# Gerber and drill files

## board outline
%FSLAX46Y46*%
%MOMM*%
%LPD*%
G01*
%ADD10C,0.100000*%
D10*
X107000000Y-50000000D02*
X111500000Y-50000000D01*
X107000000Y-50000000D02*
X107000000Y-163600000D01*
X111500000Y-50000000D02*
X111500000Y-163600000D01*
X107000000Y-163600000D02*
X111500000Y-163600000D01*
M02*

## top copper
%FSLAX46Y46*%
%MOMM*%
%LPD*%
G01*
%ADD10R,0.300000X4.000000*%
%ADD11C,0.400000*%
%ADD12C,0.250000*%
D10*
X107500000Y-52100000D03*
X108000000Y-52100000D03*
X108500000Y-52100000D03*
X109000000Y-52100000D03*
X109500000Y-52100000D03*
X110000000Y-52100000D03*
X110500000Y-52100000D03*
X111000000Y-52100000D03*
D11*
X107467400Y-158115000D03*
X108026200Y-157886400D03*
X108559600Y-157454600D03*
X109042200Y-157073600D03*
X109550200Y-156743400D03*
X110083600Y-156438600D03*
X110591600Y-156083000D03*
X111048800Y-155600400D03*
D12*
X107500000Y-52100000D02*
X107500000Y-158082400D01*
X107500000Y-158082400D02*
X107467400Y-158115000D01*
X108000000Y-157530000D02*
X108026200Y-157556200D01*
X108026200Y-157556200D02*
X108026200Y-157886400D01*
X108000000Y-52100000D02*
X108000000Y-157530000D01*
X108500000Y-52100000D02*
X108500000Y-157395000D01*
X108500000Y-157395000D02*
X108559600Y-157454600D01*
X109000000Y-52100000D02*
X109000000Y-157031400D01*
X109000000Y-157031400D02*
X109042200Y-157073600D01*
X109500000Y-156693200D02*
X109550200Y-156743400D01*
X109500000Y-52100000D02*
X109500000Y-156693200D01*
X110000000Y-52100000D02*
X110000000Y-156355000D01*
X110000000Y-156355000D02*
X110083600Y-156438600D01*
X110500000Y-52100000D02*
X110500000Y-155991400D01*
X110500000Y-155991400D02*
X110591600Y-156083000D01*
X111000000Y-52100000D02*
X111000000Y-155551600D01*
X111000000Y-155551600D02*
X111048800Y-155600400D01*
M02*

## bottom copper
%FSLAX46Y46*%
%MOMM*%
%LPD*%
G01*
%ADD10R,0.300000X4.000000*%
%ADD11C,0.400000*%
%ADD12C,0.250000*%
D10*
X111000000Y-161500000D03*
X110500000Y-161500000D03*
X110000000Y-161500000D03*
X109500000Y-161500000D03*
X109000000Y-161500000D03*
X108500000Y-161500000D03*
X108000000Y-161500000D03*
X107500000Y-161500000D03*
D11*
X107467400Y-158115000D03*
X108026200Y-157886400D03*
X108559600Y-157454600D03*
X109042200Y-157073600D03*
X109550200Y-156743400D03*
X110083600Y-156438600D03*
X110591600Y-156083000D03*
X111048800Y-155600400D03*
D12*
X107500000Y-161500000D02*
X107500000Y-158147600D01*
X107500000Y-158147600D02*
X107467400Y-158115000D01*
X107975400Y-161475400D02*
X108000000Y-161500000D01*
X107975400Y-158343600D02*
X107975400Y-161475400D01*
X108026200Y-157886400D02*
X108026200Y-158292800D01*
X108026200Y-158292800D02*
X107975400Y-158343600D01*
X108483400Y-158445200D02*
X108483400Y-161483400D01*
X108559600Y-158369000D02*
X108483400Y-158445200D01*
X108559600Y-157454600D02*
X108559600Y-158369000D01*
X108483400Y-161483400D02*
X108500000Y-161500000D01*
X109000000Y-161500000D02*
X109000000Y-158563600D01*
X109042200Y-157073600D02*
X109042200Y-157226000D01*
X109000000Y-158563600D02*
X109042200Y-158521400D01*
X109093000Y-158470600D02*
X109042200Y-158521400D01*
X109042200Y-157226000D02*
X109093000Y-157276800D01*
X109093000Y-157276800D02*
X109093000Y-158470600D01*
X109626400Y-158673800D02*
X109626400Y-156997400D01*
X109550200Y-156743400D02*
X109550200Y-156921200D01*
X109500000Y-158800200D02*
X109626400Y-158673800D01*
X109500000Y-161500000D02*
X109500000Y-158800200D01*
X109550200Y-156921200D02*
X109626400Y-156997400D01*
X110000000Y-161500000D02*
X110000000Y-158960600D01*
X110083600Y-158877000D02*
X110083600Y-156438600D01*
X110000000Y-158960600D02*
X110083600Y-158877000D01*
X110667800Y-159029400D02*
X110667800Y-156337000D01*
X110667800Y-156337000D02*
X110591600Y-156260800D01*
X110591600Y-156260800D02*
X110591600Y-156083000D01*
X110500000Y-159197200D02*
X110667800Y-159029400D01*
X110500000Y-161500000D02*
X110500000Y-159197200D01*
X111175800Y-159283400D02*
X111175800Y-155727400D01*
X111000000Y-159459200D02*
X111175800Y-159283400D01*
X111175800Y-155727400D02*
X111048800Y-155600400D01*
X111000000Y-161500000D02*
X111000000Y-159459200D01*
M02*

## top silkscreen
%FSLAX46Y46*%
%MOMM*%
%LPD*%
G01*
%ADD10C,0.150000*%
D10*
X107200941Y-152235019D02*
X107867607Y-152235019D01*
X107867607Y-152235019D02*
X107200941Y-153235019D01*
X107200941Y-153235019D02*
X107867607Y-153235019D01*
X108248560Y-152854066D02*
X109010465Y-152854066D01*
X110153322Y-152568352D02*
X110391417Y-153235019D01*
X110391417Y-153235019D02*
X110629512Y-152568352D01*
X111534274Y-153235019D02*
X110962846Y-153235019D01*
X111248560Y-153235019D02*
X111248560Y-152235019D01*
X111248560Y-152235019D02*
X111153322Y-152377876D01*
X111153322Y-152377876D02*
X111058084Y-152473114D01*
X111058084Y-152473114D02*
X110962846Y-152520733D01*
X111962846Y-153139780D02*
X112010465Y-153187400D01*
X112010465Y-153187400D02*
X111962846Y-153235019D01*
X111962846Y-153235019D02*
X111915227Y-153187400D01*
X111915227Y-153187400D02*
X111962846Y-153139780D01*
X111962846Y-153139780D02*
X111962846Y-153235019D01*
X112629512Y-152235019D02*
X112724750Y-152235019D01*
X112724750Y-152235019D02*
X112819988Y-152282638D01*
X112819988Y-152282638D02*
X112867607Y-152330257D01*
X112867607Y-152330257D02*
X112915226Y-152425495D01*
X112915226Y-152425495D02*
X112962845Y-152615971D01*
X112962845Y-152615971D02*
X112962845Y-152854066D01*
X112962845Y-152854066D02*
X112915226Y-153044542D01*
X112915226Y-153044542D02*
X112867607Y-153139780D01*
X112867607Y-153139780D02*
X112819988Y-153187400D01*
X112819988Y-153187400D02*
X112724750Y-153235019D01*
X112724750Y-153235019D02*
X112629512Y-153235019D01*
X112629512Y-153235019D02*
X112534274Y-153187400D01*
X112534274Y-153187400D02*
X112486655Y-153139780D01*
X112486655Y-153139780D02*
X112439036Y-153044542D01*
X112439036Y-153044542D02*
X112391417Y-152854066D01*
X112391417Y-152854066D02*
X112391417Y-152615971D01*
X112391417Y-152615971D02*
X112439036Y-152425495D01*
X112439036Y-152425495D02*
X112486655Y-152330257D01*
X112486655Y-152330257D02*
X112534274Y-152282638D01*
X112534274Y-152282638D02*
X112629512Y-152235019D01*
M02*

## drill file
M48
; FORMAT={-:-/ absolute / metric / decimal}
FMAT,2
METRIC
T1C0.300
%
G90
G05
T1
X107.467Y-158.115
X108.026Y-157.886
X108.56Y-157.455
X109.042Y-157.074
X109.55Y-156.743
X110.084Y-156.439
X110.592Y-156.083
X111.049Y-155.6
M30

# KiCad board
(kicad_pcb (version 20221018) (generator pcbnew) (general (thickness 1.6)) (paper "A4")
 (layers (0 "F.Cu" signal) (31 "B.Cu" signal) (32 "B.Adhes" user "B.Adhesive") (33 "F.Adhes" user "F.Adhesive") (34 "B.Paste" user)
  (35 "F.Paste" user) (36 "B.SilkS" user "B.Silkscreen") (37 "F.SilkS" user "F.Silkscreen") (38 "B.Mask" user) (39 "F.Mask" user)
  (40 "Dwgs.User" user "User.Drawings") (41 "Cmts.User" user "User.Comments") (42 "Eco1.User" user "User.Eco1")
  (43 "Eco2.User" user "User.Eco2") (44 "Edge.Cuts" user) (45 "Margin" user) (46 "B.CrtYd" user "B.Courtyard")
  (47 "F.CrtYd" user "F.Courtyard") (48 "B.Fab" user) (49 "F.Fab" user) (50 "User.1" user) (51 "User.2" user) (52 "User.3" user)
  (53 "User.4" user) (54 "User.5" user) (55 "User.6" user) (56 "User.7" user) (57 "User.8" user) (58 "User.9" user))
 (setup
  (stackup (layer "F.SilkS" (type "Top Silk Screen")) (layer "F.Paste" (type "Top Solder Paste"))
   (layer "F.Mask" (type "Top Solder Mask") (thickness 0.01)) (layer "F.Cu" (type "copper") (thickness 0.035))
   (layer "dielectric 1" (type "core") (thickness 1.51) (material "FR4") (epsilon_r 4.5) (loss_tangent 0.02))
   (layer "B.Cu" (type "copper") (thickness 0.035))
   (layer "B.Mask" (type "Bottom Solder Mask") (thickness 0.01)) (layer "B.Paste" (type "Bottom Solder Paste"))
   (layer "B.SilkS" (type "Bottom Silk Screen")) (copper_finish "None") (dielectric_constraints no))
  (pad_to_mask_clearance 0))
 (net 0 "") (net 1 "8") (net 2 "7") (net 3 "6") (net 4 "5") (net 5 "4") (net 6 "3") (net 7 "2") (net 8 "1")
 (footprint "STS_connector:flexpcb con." (layer "F.Cu") (at 107 54.1)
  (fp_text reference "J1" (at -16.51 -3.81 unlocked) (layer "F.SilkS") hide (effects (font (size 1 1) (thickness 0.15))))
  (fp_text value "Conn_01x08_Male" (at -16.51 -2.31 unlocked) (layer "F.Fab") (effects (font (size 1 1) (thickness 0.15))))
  (pad "1" smd rect (at 0.5 -2) (size 0.3 4) (layers "F.Cu" "F.Paste" "F.Mask") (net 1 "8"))
  (pad "2" smd rect (at 1 -2) (size 0.3 4) (layers "F.Cu" "F.Paste" "F.Mask") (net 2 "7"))
  (pad "3" smd rect (at 1.5 -2) (size 0.3 4) (layers "F.Cu" "F.Paste" "F.Mask") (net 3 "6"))
  (pad "4" smd rect (at 2 -2) (size 0.3 4) (layers "F.Cu" "F.Paste" "F.Mask") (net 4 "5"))
  (pad "5" smd rect (at 2.5 -2) (size 0.3 4) (layers "F.Cu" "F.Paste" "F.Mask") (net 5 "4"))
  (pad "6" smd rect (at 3 -2) (size 0.3 4) (layers "F.Cu" "F.Paste" "F.Mask") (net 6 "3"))
  (pad "7" smd rect (at 3.5 -2) (size 0.3 4) (layers "F.Cu" "F.Paste" "F.Mask") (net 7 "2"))
  (pad "8" smd rect (at 4 -2) (size 0.3 4) (layers "F.Cu" "F.Paste" "F.Mask") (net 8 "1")))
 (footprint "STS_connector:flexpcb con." (layer "B.Cu") (at 111.5 163.5 180)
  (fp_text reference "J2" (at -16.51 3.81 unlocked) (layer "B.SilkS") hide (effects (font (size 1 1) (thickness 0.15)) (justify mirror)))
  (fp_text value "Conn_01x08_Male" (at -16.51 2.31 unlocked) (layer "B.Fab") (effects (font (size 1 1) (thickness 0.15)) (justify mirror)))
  (pad "1" smd rect (at 0.5 2 180) (size 0.3 4) (layers "B.Cu" "B.Paste" "B.Mask") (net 8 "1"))
  (pad "2" smd rect (at 1 2 180) (size 0.3 4) (layers "B.Cu" "B.Paste" "B.Mask") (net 7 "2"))
  (pad "3" smd rect (at 1.5 2 180) (size 0.3 4) (layers "B.Cu" "B.Paste" "B.Mask") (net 6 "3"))
  (pad "4" smd rect (at 2 2 180) (size 0.3 4) (layers "B.Cu" "B.Paste" "B.Mask") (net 5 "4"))
  (pad "5" smd rect (at 2.5 2 180) (size 0.3 4) (layers "B.Cu" "B.Paste" "B.Mask") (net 4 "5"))
  (pad "6" smd rect (at 3 2 180) (size 0.3 4) (layers "B.Cu" "B.Paste" "B.Mask") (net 3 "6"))
  (pad "7" smd rect (at 3.5 2 180) (size 0.3 4) (layers "B.Cu" "B.Paste" "B.Mask") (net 2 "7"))
  (pad "8" smd rect (at 4 2 180) (size 0.3 4) (layers "B.Cu" "B.Paste" "B.Mask") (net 1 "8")))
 (gr_line (start 107 50) (end 111.5 50) (stroke (width 0.1) (type solid)) (layer "Edge.Cuts"))
 (gr_line (start 107 50) (end 107 163.6) (stroke (width 0.1) (type solid)) (layer "Edge.Cuts"))
 (gr_line (start 111.5 50) (end 111.5 163.6) (stroke (width 0.1) (type solid)) (layer "Edge.Cuts"))
 (gr_line (start 107 163.6) (end 111.5 163.6) (stroke (width 0.1) (type solid)) (layer "Edge.Cuts"))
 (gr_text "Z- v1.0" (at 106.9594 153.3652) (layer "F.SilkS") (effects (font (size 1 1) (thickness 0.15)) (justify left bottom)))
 (segment (start 107.5 52.1) (end 107.5 158.0824) (width 0.25) (layer "F.Cu") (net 1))
 (segment (start 107.5 158.0824) (end 107.4674 158.115) (width 0.25) (layer "F.Cu") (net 1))
 (via (at 107.4674 158.115) (size 0.4) (drill 0.3) (layers "F.Cu" "B.Cu") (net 1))
 (segment (start 107.5 161.5) (end 107.5 158.1476) (width 0.25) (layer "B.Cu") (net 1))
 (segment (start 107.5 158.1476) (end 107.4674 158.115) (width 0.25) (layer "B.Cu") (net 1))
 (segment (start 108 157.53) (end 108.0262 157.5562) (width 0.25) (layer "F.Cu") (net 2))
 (segment (start 108.0262 157.5562) (end 108.0262 157.8864) (width 0.25) (layer "F.Cu") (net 2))
 (segment (start 108 52.1) (end 108 157.53) (width 0.25) (layer "F.Cu") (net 2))
 (via (at 108.0262 157.8864) (size 0.4) (drill 0.3) (layers "F.Cu" "B.Cu") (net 2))
 (segment (start 107.9754 161.4754) (end 108 161.5) (width 0.25) (layer "B.Cu") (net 2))
 (segment (start 107.9754 158.3436) (end 107.9754 161.4754) (width 0.25) (layer "B.Cu") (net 2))
 (segment (start 108.0262 157.8864) (end 108.0262 158.2928) (width 0.25) (layer "B.Cu") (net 2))
 (segment (start 108.0262 158.2928) (end 107.9754 158.3436) (width 0.25) (layer "B.Cu") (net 2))
 (segment (start 108.5 52.1) (end 108.5 157.395) (width 0.25) (layer "F.Cu") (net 3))
 (segment (start 108.5 157.395) (end 108.5596 157.4546) (width 0.25) (layer "F.Cu") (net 3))
 (via (at 108.5596 157.4546) (size 0.4) (drill 0.3) (layers "F.Cu" "B.Cu") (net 3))
 (segment (start 108.4834 158.4452) (end 108.4834 161.4834) (width 0.25) (layer "B.Cu") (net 3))
 (segment (start 108.5596 158.369) (end 108.4834 158.4452) (width 0.25) (layer "B.Cu") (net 3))
 (segment (start 108.5596 157.4546) (end 108.5596 158.369) (width 0.25) (layer "B.Cu") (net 3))
 (segment (start 108.4834 161.4834) (end 108.5 161.5) (width 0.25) (layer "B.Cu") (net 3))
 (segment (start 109 52.1) (end 109 157.0314) (width 0.25) (layer "F.Cu") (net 4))
 (segment (start 109 157.0314) (end 109.0422 157.0736) (width 0.25) (layer "F.Cu") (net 4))
 (via (at 109.0422 157.0736) (size 0.4) (drill 0.3) (layers "F.Cu" "B.Cu") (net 4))
 (segment (start 109 161.5) (end 109 158.5636) (width 0.25) (layer "B.Cu") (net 4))
 (segment (start 109.0422 157.0736) (end 109.0422 157.226) (width 0.25) (layer "B.Cu") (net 4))
 (segment (start 109 158.5636) (end 109.0422 158.5214) (width 0.25) (layer "B.Cu") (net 4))
 (segment (start 109.093 158.4706) (end 109.0422 158.5214) (width 0.25) (layer "B.Cu") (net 4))
 (segment (start 109.0422 157.226) (end 109.093 157.2768) (width 0.25) (layer "B.Cu") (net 4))
 (segment (start 109.093 157.2768) (end 109.093 158.4706) (width 0.25) (layer "B.Cu") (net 4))
 (segment (start 109.5 156.6932) (end 109.5502 156.7434) (width 0.25) (layer "F.Cu") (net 5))
 (segment (start 109.5 52.1) (end 109.5 156.6932) (width 0.25) (layer "F.Cu") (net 5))
 (via (at 109.5502 156.7434) (size 0.4) (drill 0.3) (layers "F.Cu" "B.Cu") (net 5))
 (segment (start 109.6264 158.6738) (end 109.6264 156.9974) (width 0.25) (layer "B.Cu") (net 5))
 (segment (start 109.5502 156.7434) (end 109.5502 156.9212) (width 0.25) (layer "B.Cu") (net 5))
 (segment (start 109.5 158.8002) (end 109.6264 158.6738) (width 0.25) (layer "B.Cu") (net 5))
 (segment (start 109.5 161.5) (end 109.5 158.8002) (width 0.25) (layer "B.Cu") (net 5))
 (segment (start 109.5502 156.9212) (end 109.6264 156.9974) (width 0.25) (layer "B.Cu") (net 5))
 (segment (start 110 52.1) (end 110 156.355) (width 0.25) (layer "F.Cu") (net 6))
 (segment (start 110 156.355) (end 110.0836 156.4386) (width 0.25) (layer "F.Cu") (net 6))
 (via (at 110.0836 156.4386) (size 0.4) (drill 0.3) (layers "F.Cu" "B.Cu") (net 6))
 (segment (start 110 161.5) (end 110 158.9606) (width 0.25) (layer "B.Cu") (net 6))
 (segment (start 110.0836 158.877) (end 110.0836 156.4386) (width 0.25) (layer "B.Cu") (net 6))
 (segment (start 110 158.9606) (end 110.0836 158.877) (width 0.25) (layer "B.Cu") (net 6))
 (segment (start 110.5 52.1) (end 110.5 155.9914) (width 0.25) (layer "F.Cu") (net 7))
 (segment (start 110.5 155.9914) (end 110.5916 156.083) (width 0.25) (layer "F.Cu") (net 7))
 (via (at 110.5916 156.083) (size 0.4) (drill 0.3) (layers "F.Cu" "B.Cu") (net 7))
 (segment (start 110.6678 159.0294) (end 110.6678 156.337) (width 0.25) (layer "B.Cu") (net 7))
 (segment (start 110.6678 156.337) (end 110.5916 156.2608) (width 0.25) (layer "B.Cu") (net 7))
 (segment (start 110.5916 156.2608) (end 110.5916 156.083) (width 0.25) (layer "B.Cu") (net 7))
 (segment (start 110.5 159.1972) (end 110.6678 159.0294) (width 0.25) (layer "B.Cu") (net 7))
 (segment (start 110.5 161.5) (end 110.5 159.1972) (width 0.25) (layer "B.Cu") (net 7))
 (segment (start 111 52.1) (end 111 155.5516) (width 0.25) (layer "F.Cu") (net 8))
 (segment (start 111 155.5516) (end 111.0488 155.6004) (width 0.25) (layer "F.Cu") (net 8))
 (via (at 111.0488 155.6004) (size 0.4) (drill 0.3) (layers "F.Cu" "B.Cu") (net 8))
 (segment (start 111.1758 159.2834) (end 111.1758 155.7274) (width 0.25) (layer "B.Cu") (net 8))
 (segment (start 111 159.4592) (end 111.1758 159.2834) (width 0.25) (layer "B.Cu") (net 8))
 (segment (start 111.1758 155.7274) (end 111.0488 155.6004) (width 0.25) (layer "B.Cu") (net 8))
 (segment (start 111 161.5) (end 111 159.4592) (width 0.25) (layer "B.Cu") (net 8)))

